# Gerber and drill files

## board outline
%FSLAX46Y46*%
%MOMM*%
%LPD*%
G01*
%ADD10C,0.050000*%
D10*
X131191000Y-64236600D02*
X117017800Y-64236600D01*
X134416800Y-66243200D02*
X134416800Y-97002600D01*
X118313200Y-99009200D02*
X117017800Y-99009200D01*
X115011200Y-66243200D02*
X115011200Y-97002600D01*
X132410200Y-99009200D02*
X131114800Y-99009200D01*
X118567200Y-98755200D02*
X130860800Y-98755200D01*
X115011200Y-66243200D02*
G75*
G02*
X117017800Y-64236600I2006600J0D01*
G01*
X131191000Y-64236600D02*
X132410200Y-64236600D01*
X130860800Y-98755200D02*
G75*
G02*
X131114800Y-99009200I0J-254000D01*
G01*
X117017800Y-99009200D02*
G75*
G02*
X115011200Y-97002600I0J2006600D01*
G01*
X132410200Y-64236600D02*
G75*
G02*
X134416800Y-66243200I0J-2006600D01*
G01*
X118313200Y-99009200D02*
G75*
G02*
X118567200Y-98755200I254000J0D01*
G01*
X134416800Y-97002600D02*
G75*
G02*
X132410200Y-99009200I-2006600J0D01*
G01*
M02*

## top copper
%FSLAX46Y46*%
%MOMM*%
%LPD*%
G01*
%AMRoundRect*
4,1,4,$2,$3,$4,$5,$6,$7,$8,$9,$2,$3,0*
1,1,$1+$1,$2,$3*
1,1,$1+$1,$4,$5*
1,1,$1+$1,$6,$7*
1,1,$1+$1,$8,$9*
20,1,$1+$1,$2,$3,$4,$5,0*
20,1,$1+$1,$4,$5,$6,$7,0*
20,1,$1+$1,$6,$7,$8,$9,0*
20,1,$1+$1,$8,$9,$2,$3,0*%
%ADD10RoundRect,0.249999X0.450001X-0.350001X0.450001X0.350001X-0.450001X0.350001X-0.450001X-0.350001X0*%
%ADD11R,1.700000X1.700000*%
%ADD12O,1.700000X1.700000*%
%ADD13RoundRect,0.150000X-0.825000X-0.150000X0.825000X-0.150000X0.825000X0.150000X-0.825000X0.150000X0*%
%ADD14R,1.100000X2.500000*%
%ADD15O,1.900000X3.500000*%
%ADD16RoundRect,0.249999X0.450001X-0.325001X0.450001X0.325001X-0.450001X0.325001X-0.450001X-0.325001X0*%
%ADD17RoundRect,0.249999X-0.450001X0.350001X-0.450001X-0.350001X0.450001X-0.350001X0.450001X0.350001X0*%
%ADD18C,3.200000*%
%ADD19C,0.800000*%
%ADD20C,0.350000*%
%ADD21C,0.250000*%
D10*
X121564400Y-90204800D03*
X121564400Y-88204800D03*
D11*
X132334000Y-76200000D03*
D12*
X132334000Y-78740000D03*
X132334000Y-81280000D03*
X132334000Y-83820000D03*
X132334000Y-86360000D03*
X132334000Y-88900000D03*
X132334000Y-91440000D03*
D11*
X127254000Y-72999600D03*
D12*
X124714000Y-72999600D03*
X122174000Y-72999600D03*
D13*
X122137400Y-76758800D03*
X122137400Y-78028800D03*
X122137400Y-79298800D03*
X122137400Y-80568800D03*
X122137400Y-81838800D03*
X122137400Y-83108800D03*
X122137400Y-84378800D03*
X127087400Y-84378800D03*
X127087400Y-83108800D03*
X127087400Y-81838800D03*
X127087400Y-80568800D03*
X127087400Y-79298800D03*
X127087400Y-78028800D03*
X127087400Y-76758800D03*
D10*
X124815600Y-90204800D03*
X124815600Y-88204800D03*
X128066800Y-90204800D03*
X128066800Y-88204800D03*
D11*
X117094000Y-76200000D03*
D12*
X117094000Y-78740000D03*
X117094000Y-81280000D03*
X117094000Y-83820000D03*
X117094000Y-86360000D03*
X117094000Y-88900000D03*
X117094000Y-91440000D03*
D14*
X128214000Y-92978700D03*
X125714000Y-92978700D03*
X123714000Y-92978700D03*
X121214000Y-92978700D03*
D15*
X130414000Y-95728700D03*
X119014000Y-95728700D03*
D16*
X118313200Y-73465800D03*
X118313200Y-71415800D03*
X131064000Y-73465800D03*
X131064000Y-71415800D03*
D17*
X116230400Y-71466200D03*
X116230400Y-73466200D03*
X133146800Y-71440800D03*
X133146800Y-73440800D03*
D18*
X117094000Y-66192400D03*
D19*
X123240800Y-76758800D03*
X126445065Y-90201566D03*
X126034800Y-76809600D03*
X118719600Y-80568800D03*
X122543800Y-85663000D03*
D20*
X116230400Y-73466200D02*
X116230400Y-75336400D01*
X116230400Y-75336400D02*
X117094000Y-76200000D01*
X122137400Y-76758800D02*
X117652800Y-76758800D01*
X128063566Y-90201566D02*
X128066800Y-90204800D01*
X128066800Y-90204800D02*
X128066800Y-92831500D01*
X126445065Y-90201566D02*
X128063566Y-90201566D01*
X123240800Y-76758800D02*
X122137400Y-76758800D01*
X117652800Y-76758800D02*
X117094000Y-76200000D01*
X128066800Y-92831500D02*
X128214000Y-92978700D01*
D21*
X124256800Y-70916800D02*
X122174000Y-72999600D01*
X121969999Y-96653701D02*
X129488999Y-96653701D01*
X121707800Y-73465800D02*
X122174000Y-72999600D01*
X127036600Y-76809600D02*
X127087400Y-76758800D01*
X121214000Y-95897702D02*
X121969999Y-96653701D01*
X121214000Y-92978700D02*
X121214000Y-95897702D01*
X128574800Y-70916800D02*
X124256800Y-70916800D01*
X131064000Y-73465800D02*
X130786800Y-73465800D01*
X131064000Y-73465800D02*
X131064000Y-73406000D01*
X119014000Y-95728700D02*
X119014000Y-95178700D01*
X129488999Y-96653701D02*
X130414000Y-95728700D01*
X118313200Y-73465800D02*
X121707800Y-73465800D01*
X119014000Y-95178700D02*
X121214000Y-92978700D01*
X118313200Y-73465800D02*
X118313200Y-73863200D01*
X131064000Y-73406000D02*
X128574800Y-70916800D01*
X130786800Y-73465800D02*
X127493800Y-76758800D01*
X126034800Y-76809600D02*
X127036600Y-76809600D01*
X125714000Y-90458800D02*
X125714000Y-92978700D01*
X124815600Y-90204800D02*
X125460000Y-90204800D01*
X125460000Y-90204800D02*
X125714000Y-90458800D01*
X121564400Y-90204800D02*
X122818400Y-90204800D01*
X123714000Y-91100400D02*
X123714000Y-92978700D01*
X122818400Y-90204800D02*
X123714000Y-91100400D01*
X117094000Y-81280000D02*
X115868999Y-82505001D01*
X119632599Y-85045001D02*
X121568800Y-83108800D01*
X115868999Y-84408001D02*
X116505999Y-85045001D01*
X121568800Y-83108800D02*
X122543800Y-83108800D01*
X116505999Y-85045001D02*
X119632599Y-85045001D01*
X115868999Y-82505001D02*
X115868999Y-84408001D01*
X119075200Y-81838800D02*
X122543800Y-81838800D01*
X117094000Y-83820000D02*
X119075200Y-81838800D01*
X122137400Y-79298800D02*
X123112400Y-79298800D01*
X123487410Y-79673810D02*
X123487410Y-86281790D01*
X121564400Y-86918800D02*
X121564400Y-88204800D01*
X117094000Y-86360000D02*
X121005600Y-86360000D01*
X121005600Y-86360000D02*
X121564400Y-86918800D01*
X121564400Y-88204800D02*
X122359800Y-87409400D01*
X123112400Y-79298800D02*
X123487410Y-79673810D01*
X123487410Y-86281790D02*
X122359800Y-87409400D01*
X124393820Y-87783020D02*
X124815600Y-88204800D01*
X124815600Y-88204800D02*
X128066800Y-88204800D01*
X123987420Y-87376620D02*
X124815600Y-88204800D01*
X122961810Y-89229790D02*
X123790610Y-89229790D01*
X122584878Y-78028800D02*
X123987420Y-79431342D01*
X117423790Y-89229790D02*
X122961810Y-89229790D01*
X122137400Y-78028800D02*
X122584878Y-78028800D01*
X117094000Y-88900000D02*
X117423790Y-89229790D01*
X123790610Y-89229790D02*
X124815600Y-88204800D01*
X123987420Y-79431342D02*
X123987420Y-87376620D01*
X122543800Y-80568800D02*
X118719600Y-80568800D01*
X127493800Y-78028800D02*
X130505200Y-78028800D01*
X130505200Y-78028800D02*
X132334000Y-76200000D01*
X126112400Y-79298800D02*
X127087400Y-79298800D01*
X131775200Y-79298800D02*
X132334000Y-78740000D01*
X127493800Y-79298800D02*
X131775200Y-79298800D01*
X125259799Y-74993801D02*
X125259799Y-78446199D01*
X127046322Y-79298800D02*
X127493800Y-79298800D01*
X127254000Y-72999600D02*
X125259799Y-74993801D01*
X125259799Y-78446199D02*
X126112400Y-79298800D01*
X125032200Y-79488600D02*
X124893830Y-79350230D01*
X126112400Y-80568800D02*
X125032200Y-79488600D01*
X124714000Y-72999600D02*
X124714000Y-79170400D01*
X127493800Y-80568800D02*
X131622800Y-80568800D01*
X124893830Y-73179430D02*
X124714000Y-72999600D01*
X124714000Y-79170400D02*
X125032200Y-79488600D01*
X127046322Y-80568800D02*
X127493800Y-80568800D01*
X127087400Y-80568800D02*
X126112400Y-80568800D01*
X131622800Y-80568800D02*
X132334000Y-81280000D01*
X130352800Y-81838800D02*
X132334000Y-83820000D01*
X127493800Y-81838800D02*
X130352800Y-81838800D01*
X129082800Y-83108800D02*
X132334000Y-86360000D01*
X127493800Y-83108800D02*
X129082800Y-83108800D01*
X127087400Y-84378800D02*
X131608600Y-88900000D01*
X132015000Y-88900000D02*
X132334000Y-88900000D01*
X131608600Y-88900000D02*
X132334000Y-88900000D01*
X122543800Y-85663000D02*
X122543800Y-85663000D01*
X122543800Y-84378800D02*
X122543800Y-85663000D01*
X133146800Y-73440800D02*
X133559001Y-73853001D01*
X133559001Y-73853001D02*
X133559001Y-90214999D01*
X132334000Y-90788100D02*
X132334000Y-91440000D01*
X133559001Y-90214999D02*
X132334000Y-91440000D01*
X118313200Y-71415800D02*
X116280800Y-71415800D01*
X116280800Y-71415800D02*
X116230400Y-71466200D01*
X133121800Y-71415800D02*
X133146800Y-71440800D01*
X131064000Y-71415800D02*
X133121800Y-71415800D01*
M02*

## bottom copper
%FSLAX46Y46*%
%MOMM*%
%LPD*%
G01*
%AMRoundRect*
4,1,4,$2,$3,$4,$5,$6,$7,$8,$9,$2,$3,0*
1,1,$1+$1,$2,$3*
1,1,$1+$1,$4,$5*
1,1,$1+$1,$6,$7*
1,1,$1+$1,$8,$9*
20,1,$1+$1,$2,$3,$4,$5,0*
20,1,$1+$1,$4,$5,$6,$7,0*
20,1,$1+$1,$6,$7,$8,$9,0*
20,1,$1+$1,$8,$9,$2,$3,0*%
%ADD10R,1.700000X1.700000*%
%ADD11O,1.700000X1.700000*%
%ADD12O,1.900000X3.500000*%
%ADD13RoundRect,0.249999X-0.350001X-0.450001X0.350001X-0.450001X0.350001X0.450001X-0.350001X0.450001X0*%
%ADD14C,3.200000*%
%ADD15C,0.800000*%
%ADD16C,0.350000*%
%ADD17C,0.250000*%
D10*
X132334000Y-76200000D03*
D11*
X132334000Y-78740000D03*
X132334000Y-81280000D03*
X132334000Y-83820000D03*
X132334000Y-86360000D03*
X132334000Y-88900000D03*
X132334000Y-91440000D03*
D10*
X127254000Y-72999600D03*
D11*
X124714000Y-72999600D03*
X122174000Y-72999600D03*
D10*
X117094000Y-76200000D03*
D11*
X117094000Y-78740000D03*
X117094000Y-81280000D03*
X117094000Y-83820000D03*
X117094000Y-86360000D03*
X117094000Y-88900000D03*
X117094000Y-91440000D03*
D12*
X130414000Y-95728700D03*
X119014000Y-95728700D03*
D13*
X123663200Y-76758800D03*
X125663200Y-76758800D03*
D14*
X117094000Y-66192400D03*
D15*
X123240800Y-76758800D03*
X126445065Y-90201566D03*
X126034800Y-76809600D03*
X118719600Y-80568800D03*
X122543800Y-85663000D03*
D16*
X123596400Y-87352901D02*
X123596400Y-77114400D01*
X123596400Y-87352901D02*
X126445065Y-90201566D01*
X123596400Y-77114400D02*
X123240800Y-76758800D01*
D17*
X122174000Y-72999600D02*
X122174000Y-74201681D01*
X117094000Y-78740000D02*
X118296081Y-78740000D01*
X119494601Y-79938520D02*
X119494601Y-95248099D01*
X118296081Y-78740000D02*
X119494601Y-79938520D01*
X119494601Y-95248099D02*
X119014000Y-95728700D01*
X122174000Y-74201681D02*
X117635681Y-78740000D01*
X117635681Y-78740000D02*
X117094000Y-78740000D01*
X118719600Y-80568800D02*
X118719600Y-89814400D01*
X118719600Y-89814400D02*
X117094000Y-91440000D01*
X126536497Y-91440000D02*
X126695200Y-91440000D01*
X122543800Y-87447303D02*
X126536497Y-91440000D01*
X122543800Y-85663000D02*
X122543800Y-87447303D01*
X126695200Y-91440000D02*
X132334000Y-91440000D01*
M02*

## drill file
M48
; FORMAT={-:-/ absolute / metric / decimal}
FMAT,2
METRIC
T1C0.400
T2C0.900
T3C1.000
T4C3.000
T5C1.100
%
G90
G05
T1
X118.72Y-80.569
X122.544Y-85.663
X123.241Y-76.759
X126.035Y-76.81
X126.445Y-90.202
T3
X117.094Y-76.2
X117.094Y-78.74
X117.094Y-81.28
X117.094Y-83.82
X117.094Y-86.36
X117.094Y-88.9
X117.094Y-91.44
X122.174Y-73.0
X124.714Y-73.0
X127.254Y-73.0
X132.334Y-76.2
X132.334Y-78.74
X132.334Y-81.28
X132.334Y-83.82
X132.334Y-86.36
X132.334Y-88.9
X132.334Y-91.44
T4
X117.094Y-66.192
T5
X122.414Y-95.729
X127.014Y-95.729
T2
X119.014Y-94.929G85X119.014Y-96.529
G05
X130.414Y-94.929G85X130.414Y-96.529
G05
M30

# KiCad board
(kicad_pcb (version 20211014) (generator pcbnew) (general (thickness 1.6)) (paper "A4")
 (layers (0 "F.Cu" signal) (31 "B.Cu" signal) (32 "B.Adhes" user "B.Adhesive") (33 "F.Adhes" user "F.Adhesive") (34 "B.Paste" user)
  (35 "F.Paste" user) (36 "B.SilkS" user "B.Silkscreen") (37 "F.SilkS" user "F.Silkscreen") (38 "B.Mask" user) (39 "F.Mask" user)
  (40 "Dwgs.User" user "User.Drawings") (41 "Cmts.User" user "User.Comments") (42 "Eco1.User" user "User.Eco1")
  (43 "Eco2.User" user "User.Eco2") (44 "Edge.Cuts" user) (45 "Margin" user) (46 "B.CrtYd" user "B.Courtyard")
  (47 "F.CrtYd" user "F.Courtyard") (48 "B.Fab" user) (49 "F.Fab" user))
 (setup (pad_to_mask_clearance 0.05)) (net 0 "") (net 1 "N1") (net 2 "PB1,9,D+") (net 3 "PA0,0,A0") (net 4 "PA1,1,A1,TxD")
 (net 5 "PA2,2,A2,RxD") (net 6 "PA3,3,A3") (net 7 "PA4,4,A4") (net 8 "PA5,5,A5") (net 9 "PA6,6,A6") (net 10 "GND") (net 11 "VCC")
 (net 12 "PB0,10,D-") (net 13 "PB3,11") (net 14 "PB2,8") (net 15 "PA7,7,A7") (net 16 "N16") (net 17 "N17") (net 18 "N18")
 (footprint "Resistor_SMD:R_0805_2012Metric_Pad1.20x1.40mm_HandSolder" (layer "F.Cu") (at 121.5644 89.2048 90)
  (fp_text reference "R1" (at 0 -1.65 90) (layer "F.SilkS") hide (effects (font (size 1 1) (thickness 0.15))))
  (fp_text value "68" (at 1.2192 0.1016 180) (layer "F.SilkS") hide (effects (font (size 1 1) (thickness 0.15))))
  (pad "1" smd roundrect locked (at -1 0 90) (size 1.2 1.4) (layers "F.Cu" "F.Paste" "F.Mask") (roundrect_rratio 0.2083325) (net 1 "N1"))
  (pad "2" smd roundrect locked (at 1 0 90) (size 1.2 1.4) (layers "F.Cu" "F.Paste" "F.Mask") (roundrect_rratio 0.2083325)
   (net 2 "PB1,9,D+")))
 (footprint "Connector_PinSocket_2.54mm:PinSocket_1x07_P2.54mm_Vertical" (layer "F.Cu") (at 132.334 76.2)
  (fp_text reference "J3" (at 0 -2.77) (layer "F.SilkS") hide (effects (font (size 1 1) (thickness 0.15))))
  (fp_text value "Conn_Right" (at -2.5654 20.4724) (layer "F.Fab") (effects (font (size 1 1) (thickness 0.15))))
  (pad "1" thru_hole rect locked (at 0 0) (size 1.7 1.7) (drill 1) (layers *.Cu *.Mask) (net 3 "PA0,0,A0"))
  (pad "2" thru_hole oval locked (at 0 2.54) (size 1.7 1.7) (drill 1) (layers *.Cu *.Mask) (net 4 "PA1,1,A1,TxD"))
  (pad "3" thru_hole oval locked (at 0 5.08) (size 1.7 1.7) (drill 1) (layers *.Cu *.Mask) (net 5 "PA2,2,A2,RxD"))
  (pad "4" thru_hole oval locked (at 0 7.62) (size 1.7 1.7) (drill 1) (layers *.Cu *.Mask) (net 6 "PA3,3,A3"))
  (pad "5" thru_hole oval locked (at 0 10.16) (size 1.7 1.7) (drill 1) (layers *.Cu *.Mask) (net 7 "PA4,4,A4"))
  (pad "6" thru_hole oval locked (at 0 12.7) (size 1.7 1.7) (drill 1) (layers *.Cu *.Mask) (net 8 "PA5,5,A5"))
  (pad "7" thru_hole oval locked (at 0 15.24) (size 1.7 1.7) (drill 1) (layers *.Cu *.Mask) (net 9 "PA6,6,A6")))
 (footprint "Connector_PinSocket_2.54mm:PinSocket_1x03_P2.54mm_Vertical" (layer "F.Cu") (at 127.254 72.9996 -90)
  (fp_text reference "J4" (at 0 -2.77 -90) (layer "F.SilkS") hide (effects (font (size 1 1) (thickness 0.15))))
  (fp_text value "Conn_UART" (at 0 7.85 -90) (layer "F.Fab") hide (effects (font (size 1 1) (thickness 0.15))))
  (pad "1" thru_hole rect locked (at 0 0 270) (size 1.7 1.7) (drill 1) (layers *.Cu *.Mask) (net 4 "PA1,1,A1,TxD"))
  (pad "2" thru_hole oval locked (at 0 2.54 270) (size 1.7 1.7) (drill 1) (layers *.Cu *.Mask) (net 5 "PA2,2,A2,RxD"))
  (pad "3" thru_hole oval locked (at 0 5.08 270) (size 1.7 1.7) (drill 1) (layers *.Cu *.Mask) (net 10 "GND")))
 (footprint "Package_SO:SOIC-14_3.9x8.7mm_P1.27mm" (layer "F.Cu") (at 124.6124 80.5688)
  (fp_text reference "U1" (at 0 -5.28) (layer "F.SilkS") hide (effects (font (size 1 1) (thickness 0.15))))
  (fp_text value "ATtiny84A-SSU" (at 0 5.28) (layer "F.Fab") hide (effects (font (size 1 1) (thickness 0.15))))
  (pad "1" smd roundrect locked (at -2.475 -3.81) (size 1.95 0.6) (layers "F.Cu" "F.Paste" "F.Mask") (roundrect_rratio 0.25) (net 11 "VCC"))
  (pad "2" smd roundrect locked (at -2.475 -2.54) (size 1.95 0.6) (layers "F.Cu" "F.Paste" "F.Mask") (roundrect_rratio 0.25)
   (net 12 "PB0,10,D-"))
  (pad "3" smd roundrect locked (at -2.475 -1.27) (size 1.95 0.6) (layers "F.Cu" "F.Paste" "F.Mask") (roundrect_rratio 0.25)
   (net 2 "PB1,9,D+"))
  (pad "4" smd roundrect locked (at -2.475 0) (size 1.95 0.6) (layers "F.Cu" "F.Paste" "F.Mask") (roundrect_rratio 0.25) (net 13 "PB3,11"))
  (pad "5" smd roundrect locked (at -2.475 1.27) (size 1.95 0.6) (layers "F.Cu" "F.Paste" "F.Mask") (roundrect_rratio 0.25) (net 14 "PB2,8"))
  (pad "6" smd roundrect locked (at -2.475 2.54) (size 1.95 0.6) (layers "F.Cu" "F.Paste" "F.Mask") (roundrect_rratio 0.25)
   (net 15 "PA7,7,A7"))
  (pad "7" smd roundrect locked (at -2.475 3.81) (size 1.95 0.6) (layers "F.Cu" "F.Paste" "F.Mask") (roundrect_rratio 0.25)
   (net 9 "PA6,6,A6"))
  (pad "8" smd roundrect locked (at 2.475 3.81) (size 1.95 0.6) (layers "F.Cu" "F.Paste" "F.Mask") (roundrect_rratio 0.25)
   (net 8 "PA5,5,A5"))
  (pad "9" smd roundrect locked (at 2.475 2.54) (size 1.95 0.6) (layers "F.Cu" "F.Paste" "F.Mask") (roundrect_rratio 0.25)
   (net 7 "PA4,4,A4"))
  (pad "10" smd roundrect locked (at 2.475 1.27) (size 1.95 0.6) (layers "F.Cu" "F.Paste" "F.Mask") (roundrect_rratio 0.25)
   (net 6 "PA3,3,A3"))
  (pad "11" smd roundrect locked (at 2.475 0) (size 1.95 0.6) (layers "F.Cu" "F.Paste" "F.Mask") (roundrect_rratio 0.25)
   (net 5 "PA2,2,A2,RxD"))
  (pad "12" smd roundrect locked (at 2.475 -1.27) (size 1.95 0.6) (layers "F.Cu" "F.Paste" "F.Mask") (roundrect_rratio 0.25)
   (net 4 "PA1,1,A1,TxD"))
  (pad "13" smd roundrect locked (at 2.475 -2.54) (size 1.95 0.6) (layers "F.Cu" "F.Paste" "F.Mask") (roundrect_rratio 0.25)
   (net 3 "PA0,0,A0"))
  (pad "14" smd roundrect locked (at 2.475 -3.81) (size 1.95 0.6) (layers "F.Cu" "F.Paste" "F.Mask") (roundrect_rratio 0.25) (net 10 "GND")))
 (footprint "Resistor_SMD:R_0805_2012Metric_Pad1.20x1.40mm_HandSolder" (layer "F.Cu") (at 124.8156 89.2048 90)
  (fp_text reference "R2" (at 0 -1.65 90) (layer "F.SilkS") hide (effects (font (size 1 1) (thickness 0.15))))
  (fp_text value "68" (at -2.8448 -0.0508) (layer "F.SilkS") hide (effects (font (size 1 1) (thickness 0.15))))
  (pad "1" smd roundrect locked (at -1 0 90) (size 1.2 1.4) (layers "F.Cu" "F.Paste" "F.Mask") (roundrect_rratio 0.2083325) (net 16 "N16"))
  (pad "2" smd roundrect locked (at 1 0 90) (size 1.2 1.4) (layers "F.Cu" "F.Paste" "F.Mask") (roundrect_rratio 0.2083325)
   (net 12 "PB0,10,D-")))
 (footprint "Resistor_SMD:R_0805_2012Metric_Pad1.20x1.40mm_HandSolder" (layer "F.Cu") (at 128.0668 89.2048 90)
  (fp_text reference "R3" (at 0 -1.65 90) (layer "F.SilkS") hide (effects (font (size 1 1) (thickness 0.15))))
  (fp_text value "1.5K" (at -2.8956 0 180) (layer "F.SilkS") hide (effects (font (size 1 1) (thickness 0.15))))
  (pad "1" smd roundrect locked (at -1 0 90) (size 1.2 1.4) (layers "F.Cu" "F.Paste" "F.Mask") (roundrect_rratio 0.2083325) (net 11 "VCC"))
  (pad "2" smd roundrect locked (at 1 0 90) (size 1.2 1.4) (layers "F.Cu" "F.Paste" "F.Mask") (roundrect_rratio 0.2083325)
   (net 12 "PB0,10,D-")))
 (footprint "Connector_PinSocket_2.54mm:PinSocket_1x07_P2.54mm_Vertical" (layer "F.Cu") (at 117.094 76.2)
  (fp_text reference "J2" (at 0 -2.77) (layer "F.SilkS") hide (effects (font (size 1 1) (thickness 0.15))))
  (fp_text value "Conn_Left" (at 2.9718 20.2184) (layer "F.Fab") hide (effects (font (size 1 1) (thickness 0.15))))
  (pad "1" thru_hole rect locked (at 0 0) (size 1.7 1.7) (drill 1) (layers *.Cu *.Mask) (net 11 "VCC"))
  (pad "2" thru_hole oval locked (at 0 2.54) (size 1.7 1.7) (drill 1) (layers *.Cu *.Mask) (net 10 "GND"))
  (pad "3" thru_hole oval locked (at 0 5.08) (size 1.7 1.7) (drill 1) (layers *.Cu *.Mask) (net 15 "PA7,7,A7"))
  (pad "4" thru_hole oval locked (at 0 7.62) (size 1.7 1.7) (drill 1) (layers *.Cu *.Mask) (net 14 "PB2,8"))
  (pad "5" thru_hole oval locked (at 0 10.16) (size 1.7 1.7) (drill 1) (layers *.Cu *.Mask) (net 2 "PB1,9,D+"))
  (pad "6" thru_hole oval locked (at 0 12.7) (size 1.7 1.7) (drill 1) (layers *.Cu *.Mask) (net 12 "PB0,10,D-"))
  (pad "7" thru_hole oval locked (at 0 15.24) (size 1.7 1.7) (drill 1) (layers *.Cu *.Mask) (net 13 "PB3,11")))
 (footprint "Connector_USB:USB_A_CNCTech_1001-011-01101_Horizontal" (layer "F.Cu") (at 124.714 102.6287 -90)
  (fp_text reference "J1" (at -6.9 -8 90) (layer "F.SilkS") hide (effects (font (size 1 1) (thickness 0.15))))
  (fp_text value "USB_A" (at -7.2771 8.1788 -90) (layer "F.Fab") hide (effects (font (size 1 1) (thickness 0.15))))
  (pad "" np_thru_hole circle locked (at -6.9 -2.3 270) (size 1.1 1.1) (drill 1.1) (layers *.Cu *.Mask))
  (pad "" np_thru_hole circle locked (at -6.9 2.3 270) (size 1.1 1.1) (drill 1.1) (layers *.Cu *.Mask))
  (pad "1" smd rect locked (at -9.65 -3.5 270) (size 2.5 1.1) (layers "F.Cu" "F.Paste" "F.Mask") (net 11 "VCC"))
  (pad "2" smd rect locked (at -9.65 -1 270) (size 2.5 1.1) (layers "F.Cu" "F.Paste" "F.Mask") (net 16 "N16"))
  (pad "3" smd rect locked (at -9.65 1 270) (size 2.5 1.1) (layers "F.Cu" "F.Paste" "F.Mask") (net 1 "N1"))
  (pad "4" smd rect locked (at -9.65 3.5 270) (size 2.5 1.1) (layers "F.Cu" "F.Paste" "F.Mask") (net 10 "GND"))
  (pad "5" thru_hole oval locked (at -6.9 -5.7 270) (size 3.5 1.9) (drill oval 2.5 0.9) (layers *.Cu *.Mask) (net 10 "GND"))
  (pad "5" thru_hole oval locked (at -6.9 5.7 270) (size 3.5 1.9) (drill oval 2.5 0.9) (layers *.Cu *.Mask) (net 10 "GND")))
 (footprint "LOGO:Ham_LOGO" (layer "F.Cu") (at 126.6444 64.0588)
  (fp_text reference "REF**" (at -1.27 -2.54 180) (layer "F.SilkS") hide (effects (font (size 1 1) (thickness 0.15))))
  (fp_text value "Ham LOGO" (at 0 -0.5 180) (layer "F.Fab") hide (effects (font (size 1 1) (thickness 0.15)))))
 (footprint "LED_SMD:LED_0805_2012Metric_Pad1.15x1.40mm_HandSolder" (layer "F.Cu") (at 118.3132 72.4408 90)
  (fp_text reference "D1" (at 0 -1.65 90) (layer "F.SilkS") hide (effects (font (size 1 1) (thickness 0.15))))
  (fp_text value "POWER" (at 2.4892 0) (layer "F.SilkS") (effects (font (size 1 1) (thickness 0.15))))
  (pad "1" smd roundrect locked (at -1.025 0 90) (size 1.15 1.4) (layers "F.Cu" "F.Paste" "F.Mask") (roundrect_rratio 0.2173904348)
   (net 10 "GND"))
  (pad "2" smd roundrect locked (at 1.025 0 90) (size 1.15 1.4) (layers "F.Cu" "F.Paste" "F.Mask") (roundrect_rratio 0.2173904348)
   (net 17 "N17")))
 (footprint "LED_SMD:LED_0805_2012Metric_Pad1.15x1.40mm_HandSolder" (layer "F.Cu") (at 131.064 72.4408 90)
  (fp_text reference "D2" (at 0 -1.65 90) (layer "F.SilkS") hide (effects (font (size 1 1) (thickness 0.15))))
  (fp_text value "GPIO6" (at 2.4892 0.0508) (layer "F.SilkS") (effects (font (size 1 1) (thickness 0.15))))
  (pad "1" smd roundrect locked (at -1.025 0 90) (size 1.15 1.4) (layers "F.Cu" "F.Paste" "F.Mask") (roundrect_rratio 0.2173904348)
   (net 10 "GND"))
  (pad "2" smd roundrect locked (at 1.025 0 90) (size 1.15 1.4) (layers "F.Cu" "F.Paste" "F.Mask") (roundrect_rratio 0.2173904348)
   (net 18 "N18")))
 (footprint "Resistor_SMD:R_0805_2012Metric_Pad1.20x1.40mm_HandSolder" (layer "F.Cu") (at 116.2304 72.4662 -90)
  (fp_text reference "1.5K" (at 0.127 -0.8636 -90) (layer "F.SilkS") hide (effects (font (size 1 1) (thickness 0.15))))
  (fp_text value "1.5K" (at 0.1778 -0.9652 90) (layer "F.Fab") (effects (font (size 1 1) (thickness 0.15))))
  (pad "1" smd roundrect locked (at -1 0 270) (size 1.2 1.4) (layers "F.Cu" "F.Paste" "F.Mask") (roundrect_rratio 0.2083325) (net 17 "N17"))
  (pad "2" smd roundrect locked (at 1 0 270) (size 1.2 1.4) (layers "F.Cu" "F.Paste" "F.Mask") (roundrect_rratio 0.2083325) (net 11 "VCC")))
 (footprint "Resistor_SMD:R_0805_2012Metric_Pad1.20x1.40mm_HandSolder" (layer "F.Cu") (at 133.1468 72.4408 -90)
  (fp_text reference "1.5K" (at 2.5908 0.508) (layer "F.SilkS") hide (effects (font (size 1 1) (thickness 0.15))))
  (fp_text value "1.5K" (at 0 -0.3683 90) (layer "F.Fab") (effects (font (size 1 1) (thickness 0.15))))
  (pad "1" smd roundrect locked (at -1 0 270) (size 1.2 1.4) (layers "F.Cu" "F.Paste" "F.Mask") (roundrect_rratio 0.2083325) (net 18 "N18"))
  (pad "2" smd roundrect locked (at 1 0 270) (size 1.2 1.4) (layers "F.Cu" "F.Paste" "F.Mask") (roundrect_rratio 0.2083325)
   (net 9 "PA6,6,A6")))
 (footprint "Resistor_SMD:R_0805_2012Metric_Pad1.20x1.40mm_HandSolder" (layer "B.Cu") (at 124.6632 76.7588)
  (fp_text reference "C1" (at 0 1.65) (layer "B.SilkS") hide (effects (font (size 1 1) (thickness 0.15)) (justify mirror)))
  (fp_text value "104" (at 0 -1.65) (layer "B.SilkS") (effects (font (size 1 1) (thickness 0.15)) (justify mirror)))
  (pad "1" smd roundrect locked (at -1 0) (size 1.2 1.4) (layers "B.Cu" "B.Paste" "B.Mask") (roundrect_rratio 0.2083325) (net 11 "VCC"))
  (pad "2" smd roundrect locked (at 1 0) (size 1.2 1.4) (layers "B.Cu" "B.Paste" "B.Mask") (roundrect_rratio 0.2083325) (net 10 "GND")))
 (gr_line (start 131.191 64.2366) (end 117.0178 64.2366) (layer "Edge.Cuts") (width 0.05))
 (gr_line (start 134.4168 66.2432) (end 134.4168 97.0026) (layer "Edge.Cuts") (width 0.05))
 (gr_line (start 118.3132 99.0092) (end 117.0178 99.0092) (layer "Edge.Cuts") (width 0.05))
 (gr_line (start 115.0112 66.2432) (end 115.0112 97.0026) (layer "Edge.Cuts") (width 0.05))
 (gr_line (start 132.4102 99.0092) (end 131.1148 99.0092) (layer "Edge.Cuts") (width 0.05))
 (gr_line (start 118.5672 98.7552) (end 130.8608 98.7552) (layer "Edge.Cuts") (width 0.05))
 (gr_arc (start 115.0112 66.2432) (mid 115.59892 64.82432) (end 117.0178 64.2366) (layer "Edge.Cuts") (width 0.05))
 (gr_line (start 131.191 64.2366) (end 132.4102 64.2366) (layer "Edge.Cuts") (width 0.05))
 (gr_arc (start 130.8608 98.7552) (mid 131.040405 98.829595) (end 131.1148 99.0092) (layer "Edge.Cuts") (width 0.05))
 (gr_arc (start 117.0178 99.0092) (mid 115.59892 98.42148) (end 115.0112 97.0026) (layer "Edge.Cuts") (width 0.05))
 (gr_arc (start 132.4102 64.2366) (mid 133.82908 64.82432) (end 134.4168 66.2432) (layer "Edge.Cuts") (width 0.05))
 (gr_arc (start 118.3132 99.0092) (mid 118.387595 98.829595) (end 118.5672 98.7552) (layer "Edge.Cuts") (width 0.05))
 (gr_arc (start 134.4168 97.0026) (mid 133.82908 98.42148) (end 132.4102 99.0092) (layer "Edge.Cuts") (width 0.05))
 (via (at 117.094 66.1924) (size 3.2) (drill 3) (layers "F.Cu" "B.Cu") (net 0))
 (segment (start 116.2304 73.4662) (end 116.2304 75.3364) (width 0.35) (layer "F.Cu") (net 11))
 (segment (start 116.2304 75.3364) (end 117.094 76.2) (width 0.35) (layer "F.Cu") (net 11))
 (segment (start 122.1374 76.7588) (end 117.6528 76.7588) (width 0.35) (layer "F.Cu") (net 11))
 (segment (start 128.063566 90.201566) (end 128.0668 90.2048) (width 0.35) (layer "F.Cu") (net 11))
 (segment (start 128.0668 90.2048) (end 128.0668 92.8315) (width 0.35) (layer "F.Cu") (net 11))
 (segment (start 126.445065 90.201566) (end 128.063566 90.201566) (width 0.35) (layer "F.Cu") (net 11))
 (segment (start 123.2408 76.7588) (end 122.1374 76.7588) (width 0.35) (layer "F.Cu") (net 11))
 (segment (start 117.6528 76.7588) (end 117.094 76.2) (width 0.35) (layer "F.Cu") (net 11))
 (segment (start 128.0668 92.8315) (end 128.214 92.9787) (width 0.35) (layer "F.Cu") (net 11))
 (via (at 123.2408 76.7588) (size 0.8) (drill 0.4) (layers "F.Cu" "B.Cu") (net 11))
 (via (at 126.445065 90.201566) (size 0.8) (drill 0.4) (layers "F.Cu" "B.Cu") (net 11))
 (segment (start 123.5964 87.352901) (end 123.5964 77.1144) (width 0.35) (layer "B.Cu") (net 11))
 (segment (start 123.5964 87.352901) (end 126.445065 90.201566) (width 0.35) (layer "B.Cu") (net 11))
 (segment (start 123.5964 77.1144) (end 123.2408 76.7588) (width 0.35) (layer "B.Cu") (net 11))
 (segment (start 124.2568 70.9168) (end 122.174 72.9996) (width 0.25) (layer "F.Cu") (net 10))
 (segment (start 121.969999 96.653701) (end 129.488999 96.653701) (width 0.25) (layer "F.Cu") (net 10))
 (segment (start 121.7078 73.4658) (end 122.174 72.9996) (width 0.25) (layer "F.Cu") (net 10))
 (segment (start 127.0366 76.8096) (end 127.0874 76.7588) (width 0.25) (layer "F.Cu") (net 10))
 (segment (start 121.214 95.897702) (end 121.969999 96.653701) (width 0.25) (layer "F.Cu") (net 10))
 (segment (start 121.214 92.9787) (end 121.214 95.897702) (width 0.25) (layer "F.Cu") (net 10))
 (segment (start 128.5748 70.9168) (end 124.2568 70.9168) (width 0.25) (layer "F.Cu") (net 10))
 (segment (start 131.064 73.4658) (end 130.7868 73.4658) (width 0.25) (layer "F.Cu") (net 10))
 (segment (start 131.064 73.4658) (end 131.064 73.406) (width 0.25) (layer "F.Cu") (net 10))
 (segment (start 119.014 95.7287) (end 119.014 95.1787) (width 0.25) (layer "F.Cu") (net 10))
 (segment (start 129.488999 96.653701) (end 130.414 95.7287) (width 0.25) (layer "F.Cu") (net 10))
 (segment (start 118.3132 73.4658) (end 121.7078 73.4658) (width 0.25) (layer "F.Cu") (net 10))
 (segment (start 119.014 95.1787) (end 121.214 92.9787) (width 0.25) (layer "F.Cu") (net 10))
 (segment (start 118.3132 73.4658) (end 118.3132 73.8632) (width 0.25) (layer "F.Cu") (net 10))
 (segment (start 131.064 73.406) (end 128.5748 70.9168) (width 0.25) (layer "F.Cu") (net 10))
 (segment (start 130.7868 73.4658) (end 127.4938 76.7588) (width 0.25) (layer "F.Cu") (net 10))
 (segment (start 126.0348 76.8096) (end 127.0366 76.8096) (width 0.25) (layer "F.Cu") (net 10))
 (via (at 126.0348 76.8096) (size 0.8) (drill 0.4) (layers "F.Cu" "B.Cu") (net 10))
 (segment (start 122.174 72.9996) (end 122.174 74.201681) (width 0.25) (layer "B.Cu") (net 10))
 (segment (start 117.094 78.74) (end 118.296081 78.74) (width 0.25) (layer "B.Cu") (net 10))
 (segment (start 119.494601 79.93852) (end 119.494601 95.248099) (width 0.25) (layer "B.Cu") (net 10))
 (segment (start 118.296081 78.74) (end 119.494601 79.93852) (width 0.25) (layer "B.Cu") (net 10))
 (segment (start 119.494601 95.248099) (end 119.014 95.7287) (width 0.25) (layer "B.Cu") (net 10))
 (segment (start 122.174 74.201681) (end 117.635681 78.74) (width 0.25) (layer "B.Cu") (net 10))
 (segment (start 117.635681 78.74) (end 117.094 78.74) (width 0.25) (layer "B.Cu") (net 10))
 (segment (start 125.714 90.4588) (end 125.714 92.9787) (width 0.25) (layer "F.Cu") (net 16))
 (segment (start 124.8156 90.2048) (end 125.46 90.2048) (width 0.25) (layer "F.Cu") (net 16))
 (segment (start 125.46 90.2048) (end 125.714 90.4588) (width 0.25) (layer "F.Cu") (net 16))
 (segment (start 121.5644 90.2048) (end 122.8184 90.2048) (width 0.25) (layer "F.Cu") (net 1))
 (segment (start 123.714 91.1004) (end 123.714 92.9787) (width 0.25) (layer "F.Cu") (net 1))
 (segment (start 122.8184 90.2048) (end 123.714 91.1004) (width 0.25) (layer "F.Cu") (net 1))
 (segment (start 117.094 81.28) (end 115.868999 82.505001) (width 0.25) (layer "F.Cu") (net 15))
 (segment (start 119.632599 85.045001) (end 121.5688 83.1088) (width 0.25) (layer "F.Cu") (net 15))
 (segment (start 115.868999 84.408001) (end 116.505999 85.045001) (width 0.25) (layer "F.Cu") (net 15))
 (segment (start 121.5688 83.1088) (end 122.5438 83.1088) (width 0.25) (layer "F.Cu") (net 15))
 (segment (start 116.505999 85.045001) (end 119.632599 85.045001) (width 0.25) (layer "F.Cu") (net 15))
 (segment (start 115.868999 82.505001) (end 115.868999 84.408001) (width 0.25) (layer "F.Cu") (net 15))
 (segment (start 119.0752 81.8388) (end 122.5438 81.8388) (width 0.25) (layer "F.Cu") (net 14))
 (segment (start 117.094 83.82) (end 119.0752 81.8388) (width 0.25) (layer "F.Cu") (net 14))
 (segment (start 122.1374 79.2988) (end 123.1124 79.2988) (width 0.25) (layer "F.Cu") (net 2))
 (segment (start 123.48741 79.67381) (end 123.48741 86.28179) (width 0.25) (layer "F.Cu") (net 2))
 (segment (start 121.5644 86.9188) (end 121.5644 88.2048) (width 0.25) (layer "F.Cu") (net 2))
 (segment (start 117.094 86.36) (end 121.0056 86.36) (width 0.25) (layer "F.Cu") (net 2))
 (segment (start 121.0056 86.36) (end 121.5644 86.9188) (width 0.25) (layer "F.Cu") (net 2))
 (segment (start 121.5644 88.2048) (end 122.3598 87.4094) (width 0.25) (layer "F.Cu") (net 2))
 (segment (start 123.1124 79.2988) (end 123.48741 79.67381) (width 0.25) (layer "F.Cu") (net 2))
 (segment (start 123.48741 86.28179) (end 122.3598 87.4094) (width 0.25) (layer "F.Cu") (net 2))
 (segment (start 124.39382 87.78302) (end 124.8156 88.2048) (width 0.25) (layer "F.Cu") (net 12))
 (segment (start 124.8156 88.2048) (end 128.0668 88.2048) (width 0.25) (layer "F.Cu") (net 12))
 (segment (start 123.98742 87.37662) (end 124.8156 88.2048) (width 0.25) (layer "F.Cu") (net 12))
 (segment (start 122.96181 89.22979) (end 123.79061 89.22979) (width 0.25) (layer "F.Cu") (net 12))
 (segment (start 122.584878 78.0288) (end 123.98742 79.431342) (width 0.25) (layer "F.Cu") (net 12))
 (segment (start 117.42379 89.22979) (end 122.96181 89.22979) (width 0.25) (layer "F.Cu") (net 12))
 (segment (start 122.1374 78.0288) (end 122.584878 78.0288) (width 0.25) (layer "F.Cu") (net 12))
 (segment (start 117.094 88.9) (end 117.42379 89.22979) (width 0.25) (layer "F.Cu") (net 12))
 (segment (start 123.79061 89.22979) (end 124.8156 88.2048) (width 0.25) (layer "F.Cu") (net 12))
 (segment (start 123.98742 79.431342) (end 123.98742 87.37662) (width 0.25) (layer "F.Cu") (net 12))
 (segment (start 122.5438 80.5688) (end 118.7196 80.5688) (width 0.25) (layer "F.Cu") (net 13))
 (via (at 118.7196 80.5688) (size 0.8) (drill 0.4) (layers "F.Cu" "B.Cu") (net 13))
 (segment (start 118.7196 80.5688) (end 118.7196 89.8144) (width 0.25) (layer "B.Cu") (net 13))
 (segment (start 118.7196 89.8144) (end 117.094 91.44) (width 0.25) (layer "B.Cu") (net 13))
 (segment (start 127.4938 78.0288) (end 130.5052 78.0288) (width 0.25) (layer "F.Cu") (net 3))
 (segment (start 130.5052 78.0288) (end 132.334 76.2) (width 0.25) (layer "F.Cu") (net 3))
 (segment (start 126.1124 79.2988) (end 127.0874 79.2988) (width 0.25) (layer "F.Cu") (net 4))
 (segment (start 131.7752 79.2988) (end 132.334 78.74) (width 0.25) (layer "F.Cu") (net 4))
 (segment (start 127.4938 79.2988) (end 131.7752 79.2988) (width 0.25) (layer "F.Cu") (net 4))
 (segment (start 125.259799 74.993801) (end 125.259799 78.446199) (width 0.25) (layer "F.Cu") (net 4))
 (segment (start 127.046322 79.2988) (end 127.4938 79.2988) (width 0.25) (layer "F.Cu") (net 4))
 (segment (start 127.254 72.9996) (end 125.259799 74.993801) (width 0.25) (layer "F.Cu") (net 4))
 (segment (start 125.259799 78.446199) (end 126.1124 79.2988) (width 0.25) (layer "F.Cu") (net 4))
 (segment (start 125.0322 79.4886) (end 124.89383 79.35023) (width 0.25) (layer "F.Cu") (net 5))
 (segment (start 126.1124 80.5688) (end 125.0322 79.4886) (width 0.25) (layer "F.Cu") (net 5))
 (segment (start 124.714 72.9996) (end 124.714 79.1704) (width 0.25) (layer "F.Cu") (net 5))
 (segment (start 127.4938 80.5688) (end 131.6228 80.5688) (width 0.25) (layer "F.Cu") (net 5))
 (segment (start 124.89383 73.17943) (end 124.714 72.9996) (width 0.25) (layer "F.Cu") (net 5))
 (segment (start 124.714 79.1704) (end 125.0322 79.4886) (width 0.25) (layer "F.Cu") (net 5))
 (segment (start 127.046322 80.5688) (end 127.4938 80.5688) (width 0.25) (layer "F.Cu") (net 5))
 (segment (start 127.0874 80.5688) (end 126.1124 80.5688) (width 0.25) (layer "F.Cu") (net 5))
 (segment (start 131.6228 80.5688) (end 132.334 81.28) (width 0.25) (layer "F.Cu") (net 5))
 (segment (start 130.3528 81.8388) (end 132.334 83.82) (width 0.25) (layer "F.Cu") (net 6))
 (segment (start 127.4938 81.8388) (end 130.3528 81.8388) (width 0.25) (layer "F.Cu") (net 6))
 (segment (start 129.0828 83.1088) (end 132.334 86.36) (width 0.25) (layer "F.Cu") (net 7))
 (segment (start 127.4938 83.1088) (end 129.0828 83.1088) (width 0.25) (layer "F.Cu") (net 7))
 (segment (start 127.0874 84.3788) (end 131.6086 88.9) (width 0.25) (layer "F.Cu") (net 8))
 (segment (start 132.015 88.9) (end 132.334 88.9) (width 0.25) (layer "F.Cu") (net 8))
 (segment (start 131.6086 88.9) (end 132.334 88.9) (width 0.25) (layer "F.Cu") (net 8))
 (segment (start 122.5438 85.663) (end 122.5438 85.663) (width 0.25) (layer "F.Cu") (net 9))
 (segment (start 122.5438 84.3788) (end 122.5438 85.663) (width 0.25) (layer "F.Cu") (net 9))
 (segment (start 133.1468 73.4408) (end 133.559001 73.853001) (width 0.25) (layer "F.Cu") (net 9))
 (segment (start 133.559001 73.853001) (end 133.559001 90.214999) (width 0.25) (layer "F.Cu") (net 9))
 (segment (start 132.334 90.7881) (end 132.334 91.44) (width 0.25) (layer "F.Cu") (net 9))
 (segment (start 133.559001 90.214999) (end 132.334 91.44) (width 0.25) (layer "F.Cu") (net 9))
 (via (at 122.5438 85.663) (size 0.8) (drill 0.4) (layers "F.Cu" "B.Cu") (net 9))
 (segment (start 126.536497 91.44) (end 126.6952 91.44) (width 0.25) (layer "B.Cu") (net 9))
 (segment (start 122.5438 87.447303) (end 126.536497 91.44) (width 0.25) (layer "B.Cu") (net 9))
 (segment (start 122.5438 85.663) (end 122.5438 87.447303) (width 0.25) (layer "B.Cu") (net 9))
 (segment (start 126.6952 91.44) (end 132.334 91.44) (width 0.25) (layer "B.Cu") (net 9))
 (segment (start 118.3132 71.4158) (end 116.2808 71.4158) (width 0.25) (layer "F.Cu") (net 17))
 (segment (start 116.2808 71.4158) (end 116.2304 71.4662) (width 0.25) (layer "F.Cu") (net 17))
 (segment (start 133.1218 71.4158) (end 133.1468 71.4408) (width 0.25) (layer "F.Cu") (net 18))
 (segment (start 131.064 71.4158) (end 133.1218 71.4158) (width 0.25) (layer "F.Cu") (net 18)))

